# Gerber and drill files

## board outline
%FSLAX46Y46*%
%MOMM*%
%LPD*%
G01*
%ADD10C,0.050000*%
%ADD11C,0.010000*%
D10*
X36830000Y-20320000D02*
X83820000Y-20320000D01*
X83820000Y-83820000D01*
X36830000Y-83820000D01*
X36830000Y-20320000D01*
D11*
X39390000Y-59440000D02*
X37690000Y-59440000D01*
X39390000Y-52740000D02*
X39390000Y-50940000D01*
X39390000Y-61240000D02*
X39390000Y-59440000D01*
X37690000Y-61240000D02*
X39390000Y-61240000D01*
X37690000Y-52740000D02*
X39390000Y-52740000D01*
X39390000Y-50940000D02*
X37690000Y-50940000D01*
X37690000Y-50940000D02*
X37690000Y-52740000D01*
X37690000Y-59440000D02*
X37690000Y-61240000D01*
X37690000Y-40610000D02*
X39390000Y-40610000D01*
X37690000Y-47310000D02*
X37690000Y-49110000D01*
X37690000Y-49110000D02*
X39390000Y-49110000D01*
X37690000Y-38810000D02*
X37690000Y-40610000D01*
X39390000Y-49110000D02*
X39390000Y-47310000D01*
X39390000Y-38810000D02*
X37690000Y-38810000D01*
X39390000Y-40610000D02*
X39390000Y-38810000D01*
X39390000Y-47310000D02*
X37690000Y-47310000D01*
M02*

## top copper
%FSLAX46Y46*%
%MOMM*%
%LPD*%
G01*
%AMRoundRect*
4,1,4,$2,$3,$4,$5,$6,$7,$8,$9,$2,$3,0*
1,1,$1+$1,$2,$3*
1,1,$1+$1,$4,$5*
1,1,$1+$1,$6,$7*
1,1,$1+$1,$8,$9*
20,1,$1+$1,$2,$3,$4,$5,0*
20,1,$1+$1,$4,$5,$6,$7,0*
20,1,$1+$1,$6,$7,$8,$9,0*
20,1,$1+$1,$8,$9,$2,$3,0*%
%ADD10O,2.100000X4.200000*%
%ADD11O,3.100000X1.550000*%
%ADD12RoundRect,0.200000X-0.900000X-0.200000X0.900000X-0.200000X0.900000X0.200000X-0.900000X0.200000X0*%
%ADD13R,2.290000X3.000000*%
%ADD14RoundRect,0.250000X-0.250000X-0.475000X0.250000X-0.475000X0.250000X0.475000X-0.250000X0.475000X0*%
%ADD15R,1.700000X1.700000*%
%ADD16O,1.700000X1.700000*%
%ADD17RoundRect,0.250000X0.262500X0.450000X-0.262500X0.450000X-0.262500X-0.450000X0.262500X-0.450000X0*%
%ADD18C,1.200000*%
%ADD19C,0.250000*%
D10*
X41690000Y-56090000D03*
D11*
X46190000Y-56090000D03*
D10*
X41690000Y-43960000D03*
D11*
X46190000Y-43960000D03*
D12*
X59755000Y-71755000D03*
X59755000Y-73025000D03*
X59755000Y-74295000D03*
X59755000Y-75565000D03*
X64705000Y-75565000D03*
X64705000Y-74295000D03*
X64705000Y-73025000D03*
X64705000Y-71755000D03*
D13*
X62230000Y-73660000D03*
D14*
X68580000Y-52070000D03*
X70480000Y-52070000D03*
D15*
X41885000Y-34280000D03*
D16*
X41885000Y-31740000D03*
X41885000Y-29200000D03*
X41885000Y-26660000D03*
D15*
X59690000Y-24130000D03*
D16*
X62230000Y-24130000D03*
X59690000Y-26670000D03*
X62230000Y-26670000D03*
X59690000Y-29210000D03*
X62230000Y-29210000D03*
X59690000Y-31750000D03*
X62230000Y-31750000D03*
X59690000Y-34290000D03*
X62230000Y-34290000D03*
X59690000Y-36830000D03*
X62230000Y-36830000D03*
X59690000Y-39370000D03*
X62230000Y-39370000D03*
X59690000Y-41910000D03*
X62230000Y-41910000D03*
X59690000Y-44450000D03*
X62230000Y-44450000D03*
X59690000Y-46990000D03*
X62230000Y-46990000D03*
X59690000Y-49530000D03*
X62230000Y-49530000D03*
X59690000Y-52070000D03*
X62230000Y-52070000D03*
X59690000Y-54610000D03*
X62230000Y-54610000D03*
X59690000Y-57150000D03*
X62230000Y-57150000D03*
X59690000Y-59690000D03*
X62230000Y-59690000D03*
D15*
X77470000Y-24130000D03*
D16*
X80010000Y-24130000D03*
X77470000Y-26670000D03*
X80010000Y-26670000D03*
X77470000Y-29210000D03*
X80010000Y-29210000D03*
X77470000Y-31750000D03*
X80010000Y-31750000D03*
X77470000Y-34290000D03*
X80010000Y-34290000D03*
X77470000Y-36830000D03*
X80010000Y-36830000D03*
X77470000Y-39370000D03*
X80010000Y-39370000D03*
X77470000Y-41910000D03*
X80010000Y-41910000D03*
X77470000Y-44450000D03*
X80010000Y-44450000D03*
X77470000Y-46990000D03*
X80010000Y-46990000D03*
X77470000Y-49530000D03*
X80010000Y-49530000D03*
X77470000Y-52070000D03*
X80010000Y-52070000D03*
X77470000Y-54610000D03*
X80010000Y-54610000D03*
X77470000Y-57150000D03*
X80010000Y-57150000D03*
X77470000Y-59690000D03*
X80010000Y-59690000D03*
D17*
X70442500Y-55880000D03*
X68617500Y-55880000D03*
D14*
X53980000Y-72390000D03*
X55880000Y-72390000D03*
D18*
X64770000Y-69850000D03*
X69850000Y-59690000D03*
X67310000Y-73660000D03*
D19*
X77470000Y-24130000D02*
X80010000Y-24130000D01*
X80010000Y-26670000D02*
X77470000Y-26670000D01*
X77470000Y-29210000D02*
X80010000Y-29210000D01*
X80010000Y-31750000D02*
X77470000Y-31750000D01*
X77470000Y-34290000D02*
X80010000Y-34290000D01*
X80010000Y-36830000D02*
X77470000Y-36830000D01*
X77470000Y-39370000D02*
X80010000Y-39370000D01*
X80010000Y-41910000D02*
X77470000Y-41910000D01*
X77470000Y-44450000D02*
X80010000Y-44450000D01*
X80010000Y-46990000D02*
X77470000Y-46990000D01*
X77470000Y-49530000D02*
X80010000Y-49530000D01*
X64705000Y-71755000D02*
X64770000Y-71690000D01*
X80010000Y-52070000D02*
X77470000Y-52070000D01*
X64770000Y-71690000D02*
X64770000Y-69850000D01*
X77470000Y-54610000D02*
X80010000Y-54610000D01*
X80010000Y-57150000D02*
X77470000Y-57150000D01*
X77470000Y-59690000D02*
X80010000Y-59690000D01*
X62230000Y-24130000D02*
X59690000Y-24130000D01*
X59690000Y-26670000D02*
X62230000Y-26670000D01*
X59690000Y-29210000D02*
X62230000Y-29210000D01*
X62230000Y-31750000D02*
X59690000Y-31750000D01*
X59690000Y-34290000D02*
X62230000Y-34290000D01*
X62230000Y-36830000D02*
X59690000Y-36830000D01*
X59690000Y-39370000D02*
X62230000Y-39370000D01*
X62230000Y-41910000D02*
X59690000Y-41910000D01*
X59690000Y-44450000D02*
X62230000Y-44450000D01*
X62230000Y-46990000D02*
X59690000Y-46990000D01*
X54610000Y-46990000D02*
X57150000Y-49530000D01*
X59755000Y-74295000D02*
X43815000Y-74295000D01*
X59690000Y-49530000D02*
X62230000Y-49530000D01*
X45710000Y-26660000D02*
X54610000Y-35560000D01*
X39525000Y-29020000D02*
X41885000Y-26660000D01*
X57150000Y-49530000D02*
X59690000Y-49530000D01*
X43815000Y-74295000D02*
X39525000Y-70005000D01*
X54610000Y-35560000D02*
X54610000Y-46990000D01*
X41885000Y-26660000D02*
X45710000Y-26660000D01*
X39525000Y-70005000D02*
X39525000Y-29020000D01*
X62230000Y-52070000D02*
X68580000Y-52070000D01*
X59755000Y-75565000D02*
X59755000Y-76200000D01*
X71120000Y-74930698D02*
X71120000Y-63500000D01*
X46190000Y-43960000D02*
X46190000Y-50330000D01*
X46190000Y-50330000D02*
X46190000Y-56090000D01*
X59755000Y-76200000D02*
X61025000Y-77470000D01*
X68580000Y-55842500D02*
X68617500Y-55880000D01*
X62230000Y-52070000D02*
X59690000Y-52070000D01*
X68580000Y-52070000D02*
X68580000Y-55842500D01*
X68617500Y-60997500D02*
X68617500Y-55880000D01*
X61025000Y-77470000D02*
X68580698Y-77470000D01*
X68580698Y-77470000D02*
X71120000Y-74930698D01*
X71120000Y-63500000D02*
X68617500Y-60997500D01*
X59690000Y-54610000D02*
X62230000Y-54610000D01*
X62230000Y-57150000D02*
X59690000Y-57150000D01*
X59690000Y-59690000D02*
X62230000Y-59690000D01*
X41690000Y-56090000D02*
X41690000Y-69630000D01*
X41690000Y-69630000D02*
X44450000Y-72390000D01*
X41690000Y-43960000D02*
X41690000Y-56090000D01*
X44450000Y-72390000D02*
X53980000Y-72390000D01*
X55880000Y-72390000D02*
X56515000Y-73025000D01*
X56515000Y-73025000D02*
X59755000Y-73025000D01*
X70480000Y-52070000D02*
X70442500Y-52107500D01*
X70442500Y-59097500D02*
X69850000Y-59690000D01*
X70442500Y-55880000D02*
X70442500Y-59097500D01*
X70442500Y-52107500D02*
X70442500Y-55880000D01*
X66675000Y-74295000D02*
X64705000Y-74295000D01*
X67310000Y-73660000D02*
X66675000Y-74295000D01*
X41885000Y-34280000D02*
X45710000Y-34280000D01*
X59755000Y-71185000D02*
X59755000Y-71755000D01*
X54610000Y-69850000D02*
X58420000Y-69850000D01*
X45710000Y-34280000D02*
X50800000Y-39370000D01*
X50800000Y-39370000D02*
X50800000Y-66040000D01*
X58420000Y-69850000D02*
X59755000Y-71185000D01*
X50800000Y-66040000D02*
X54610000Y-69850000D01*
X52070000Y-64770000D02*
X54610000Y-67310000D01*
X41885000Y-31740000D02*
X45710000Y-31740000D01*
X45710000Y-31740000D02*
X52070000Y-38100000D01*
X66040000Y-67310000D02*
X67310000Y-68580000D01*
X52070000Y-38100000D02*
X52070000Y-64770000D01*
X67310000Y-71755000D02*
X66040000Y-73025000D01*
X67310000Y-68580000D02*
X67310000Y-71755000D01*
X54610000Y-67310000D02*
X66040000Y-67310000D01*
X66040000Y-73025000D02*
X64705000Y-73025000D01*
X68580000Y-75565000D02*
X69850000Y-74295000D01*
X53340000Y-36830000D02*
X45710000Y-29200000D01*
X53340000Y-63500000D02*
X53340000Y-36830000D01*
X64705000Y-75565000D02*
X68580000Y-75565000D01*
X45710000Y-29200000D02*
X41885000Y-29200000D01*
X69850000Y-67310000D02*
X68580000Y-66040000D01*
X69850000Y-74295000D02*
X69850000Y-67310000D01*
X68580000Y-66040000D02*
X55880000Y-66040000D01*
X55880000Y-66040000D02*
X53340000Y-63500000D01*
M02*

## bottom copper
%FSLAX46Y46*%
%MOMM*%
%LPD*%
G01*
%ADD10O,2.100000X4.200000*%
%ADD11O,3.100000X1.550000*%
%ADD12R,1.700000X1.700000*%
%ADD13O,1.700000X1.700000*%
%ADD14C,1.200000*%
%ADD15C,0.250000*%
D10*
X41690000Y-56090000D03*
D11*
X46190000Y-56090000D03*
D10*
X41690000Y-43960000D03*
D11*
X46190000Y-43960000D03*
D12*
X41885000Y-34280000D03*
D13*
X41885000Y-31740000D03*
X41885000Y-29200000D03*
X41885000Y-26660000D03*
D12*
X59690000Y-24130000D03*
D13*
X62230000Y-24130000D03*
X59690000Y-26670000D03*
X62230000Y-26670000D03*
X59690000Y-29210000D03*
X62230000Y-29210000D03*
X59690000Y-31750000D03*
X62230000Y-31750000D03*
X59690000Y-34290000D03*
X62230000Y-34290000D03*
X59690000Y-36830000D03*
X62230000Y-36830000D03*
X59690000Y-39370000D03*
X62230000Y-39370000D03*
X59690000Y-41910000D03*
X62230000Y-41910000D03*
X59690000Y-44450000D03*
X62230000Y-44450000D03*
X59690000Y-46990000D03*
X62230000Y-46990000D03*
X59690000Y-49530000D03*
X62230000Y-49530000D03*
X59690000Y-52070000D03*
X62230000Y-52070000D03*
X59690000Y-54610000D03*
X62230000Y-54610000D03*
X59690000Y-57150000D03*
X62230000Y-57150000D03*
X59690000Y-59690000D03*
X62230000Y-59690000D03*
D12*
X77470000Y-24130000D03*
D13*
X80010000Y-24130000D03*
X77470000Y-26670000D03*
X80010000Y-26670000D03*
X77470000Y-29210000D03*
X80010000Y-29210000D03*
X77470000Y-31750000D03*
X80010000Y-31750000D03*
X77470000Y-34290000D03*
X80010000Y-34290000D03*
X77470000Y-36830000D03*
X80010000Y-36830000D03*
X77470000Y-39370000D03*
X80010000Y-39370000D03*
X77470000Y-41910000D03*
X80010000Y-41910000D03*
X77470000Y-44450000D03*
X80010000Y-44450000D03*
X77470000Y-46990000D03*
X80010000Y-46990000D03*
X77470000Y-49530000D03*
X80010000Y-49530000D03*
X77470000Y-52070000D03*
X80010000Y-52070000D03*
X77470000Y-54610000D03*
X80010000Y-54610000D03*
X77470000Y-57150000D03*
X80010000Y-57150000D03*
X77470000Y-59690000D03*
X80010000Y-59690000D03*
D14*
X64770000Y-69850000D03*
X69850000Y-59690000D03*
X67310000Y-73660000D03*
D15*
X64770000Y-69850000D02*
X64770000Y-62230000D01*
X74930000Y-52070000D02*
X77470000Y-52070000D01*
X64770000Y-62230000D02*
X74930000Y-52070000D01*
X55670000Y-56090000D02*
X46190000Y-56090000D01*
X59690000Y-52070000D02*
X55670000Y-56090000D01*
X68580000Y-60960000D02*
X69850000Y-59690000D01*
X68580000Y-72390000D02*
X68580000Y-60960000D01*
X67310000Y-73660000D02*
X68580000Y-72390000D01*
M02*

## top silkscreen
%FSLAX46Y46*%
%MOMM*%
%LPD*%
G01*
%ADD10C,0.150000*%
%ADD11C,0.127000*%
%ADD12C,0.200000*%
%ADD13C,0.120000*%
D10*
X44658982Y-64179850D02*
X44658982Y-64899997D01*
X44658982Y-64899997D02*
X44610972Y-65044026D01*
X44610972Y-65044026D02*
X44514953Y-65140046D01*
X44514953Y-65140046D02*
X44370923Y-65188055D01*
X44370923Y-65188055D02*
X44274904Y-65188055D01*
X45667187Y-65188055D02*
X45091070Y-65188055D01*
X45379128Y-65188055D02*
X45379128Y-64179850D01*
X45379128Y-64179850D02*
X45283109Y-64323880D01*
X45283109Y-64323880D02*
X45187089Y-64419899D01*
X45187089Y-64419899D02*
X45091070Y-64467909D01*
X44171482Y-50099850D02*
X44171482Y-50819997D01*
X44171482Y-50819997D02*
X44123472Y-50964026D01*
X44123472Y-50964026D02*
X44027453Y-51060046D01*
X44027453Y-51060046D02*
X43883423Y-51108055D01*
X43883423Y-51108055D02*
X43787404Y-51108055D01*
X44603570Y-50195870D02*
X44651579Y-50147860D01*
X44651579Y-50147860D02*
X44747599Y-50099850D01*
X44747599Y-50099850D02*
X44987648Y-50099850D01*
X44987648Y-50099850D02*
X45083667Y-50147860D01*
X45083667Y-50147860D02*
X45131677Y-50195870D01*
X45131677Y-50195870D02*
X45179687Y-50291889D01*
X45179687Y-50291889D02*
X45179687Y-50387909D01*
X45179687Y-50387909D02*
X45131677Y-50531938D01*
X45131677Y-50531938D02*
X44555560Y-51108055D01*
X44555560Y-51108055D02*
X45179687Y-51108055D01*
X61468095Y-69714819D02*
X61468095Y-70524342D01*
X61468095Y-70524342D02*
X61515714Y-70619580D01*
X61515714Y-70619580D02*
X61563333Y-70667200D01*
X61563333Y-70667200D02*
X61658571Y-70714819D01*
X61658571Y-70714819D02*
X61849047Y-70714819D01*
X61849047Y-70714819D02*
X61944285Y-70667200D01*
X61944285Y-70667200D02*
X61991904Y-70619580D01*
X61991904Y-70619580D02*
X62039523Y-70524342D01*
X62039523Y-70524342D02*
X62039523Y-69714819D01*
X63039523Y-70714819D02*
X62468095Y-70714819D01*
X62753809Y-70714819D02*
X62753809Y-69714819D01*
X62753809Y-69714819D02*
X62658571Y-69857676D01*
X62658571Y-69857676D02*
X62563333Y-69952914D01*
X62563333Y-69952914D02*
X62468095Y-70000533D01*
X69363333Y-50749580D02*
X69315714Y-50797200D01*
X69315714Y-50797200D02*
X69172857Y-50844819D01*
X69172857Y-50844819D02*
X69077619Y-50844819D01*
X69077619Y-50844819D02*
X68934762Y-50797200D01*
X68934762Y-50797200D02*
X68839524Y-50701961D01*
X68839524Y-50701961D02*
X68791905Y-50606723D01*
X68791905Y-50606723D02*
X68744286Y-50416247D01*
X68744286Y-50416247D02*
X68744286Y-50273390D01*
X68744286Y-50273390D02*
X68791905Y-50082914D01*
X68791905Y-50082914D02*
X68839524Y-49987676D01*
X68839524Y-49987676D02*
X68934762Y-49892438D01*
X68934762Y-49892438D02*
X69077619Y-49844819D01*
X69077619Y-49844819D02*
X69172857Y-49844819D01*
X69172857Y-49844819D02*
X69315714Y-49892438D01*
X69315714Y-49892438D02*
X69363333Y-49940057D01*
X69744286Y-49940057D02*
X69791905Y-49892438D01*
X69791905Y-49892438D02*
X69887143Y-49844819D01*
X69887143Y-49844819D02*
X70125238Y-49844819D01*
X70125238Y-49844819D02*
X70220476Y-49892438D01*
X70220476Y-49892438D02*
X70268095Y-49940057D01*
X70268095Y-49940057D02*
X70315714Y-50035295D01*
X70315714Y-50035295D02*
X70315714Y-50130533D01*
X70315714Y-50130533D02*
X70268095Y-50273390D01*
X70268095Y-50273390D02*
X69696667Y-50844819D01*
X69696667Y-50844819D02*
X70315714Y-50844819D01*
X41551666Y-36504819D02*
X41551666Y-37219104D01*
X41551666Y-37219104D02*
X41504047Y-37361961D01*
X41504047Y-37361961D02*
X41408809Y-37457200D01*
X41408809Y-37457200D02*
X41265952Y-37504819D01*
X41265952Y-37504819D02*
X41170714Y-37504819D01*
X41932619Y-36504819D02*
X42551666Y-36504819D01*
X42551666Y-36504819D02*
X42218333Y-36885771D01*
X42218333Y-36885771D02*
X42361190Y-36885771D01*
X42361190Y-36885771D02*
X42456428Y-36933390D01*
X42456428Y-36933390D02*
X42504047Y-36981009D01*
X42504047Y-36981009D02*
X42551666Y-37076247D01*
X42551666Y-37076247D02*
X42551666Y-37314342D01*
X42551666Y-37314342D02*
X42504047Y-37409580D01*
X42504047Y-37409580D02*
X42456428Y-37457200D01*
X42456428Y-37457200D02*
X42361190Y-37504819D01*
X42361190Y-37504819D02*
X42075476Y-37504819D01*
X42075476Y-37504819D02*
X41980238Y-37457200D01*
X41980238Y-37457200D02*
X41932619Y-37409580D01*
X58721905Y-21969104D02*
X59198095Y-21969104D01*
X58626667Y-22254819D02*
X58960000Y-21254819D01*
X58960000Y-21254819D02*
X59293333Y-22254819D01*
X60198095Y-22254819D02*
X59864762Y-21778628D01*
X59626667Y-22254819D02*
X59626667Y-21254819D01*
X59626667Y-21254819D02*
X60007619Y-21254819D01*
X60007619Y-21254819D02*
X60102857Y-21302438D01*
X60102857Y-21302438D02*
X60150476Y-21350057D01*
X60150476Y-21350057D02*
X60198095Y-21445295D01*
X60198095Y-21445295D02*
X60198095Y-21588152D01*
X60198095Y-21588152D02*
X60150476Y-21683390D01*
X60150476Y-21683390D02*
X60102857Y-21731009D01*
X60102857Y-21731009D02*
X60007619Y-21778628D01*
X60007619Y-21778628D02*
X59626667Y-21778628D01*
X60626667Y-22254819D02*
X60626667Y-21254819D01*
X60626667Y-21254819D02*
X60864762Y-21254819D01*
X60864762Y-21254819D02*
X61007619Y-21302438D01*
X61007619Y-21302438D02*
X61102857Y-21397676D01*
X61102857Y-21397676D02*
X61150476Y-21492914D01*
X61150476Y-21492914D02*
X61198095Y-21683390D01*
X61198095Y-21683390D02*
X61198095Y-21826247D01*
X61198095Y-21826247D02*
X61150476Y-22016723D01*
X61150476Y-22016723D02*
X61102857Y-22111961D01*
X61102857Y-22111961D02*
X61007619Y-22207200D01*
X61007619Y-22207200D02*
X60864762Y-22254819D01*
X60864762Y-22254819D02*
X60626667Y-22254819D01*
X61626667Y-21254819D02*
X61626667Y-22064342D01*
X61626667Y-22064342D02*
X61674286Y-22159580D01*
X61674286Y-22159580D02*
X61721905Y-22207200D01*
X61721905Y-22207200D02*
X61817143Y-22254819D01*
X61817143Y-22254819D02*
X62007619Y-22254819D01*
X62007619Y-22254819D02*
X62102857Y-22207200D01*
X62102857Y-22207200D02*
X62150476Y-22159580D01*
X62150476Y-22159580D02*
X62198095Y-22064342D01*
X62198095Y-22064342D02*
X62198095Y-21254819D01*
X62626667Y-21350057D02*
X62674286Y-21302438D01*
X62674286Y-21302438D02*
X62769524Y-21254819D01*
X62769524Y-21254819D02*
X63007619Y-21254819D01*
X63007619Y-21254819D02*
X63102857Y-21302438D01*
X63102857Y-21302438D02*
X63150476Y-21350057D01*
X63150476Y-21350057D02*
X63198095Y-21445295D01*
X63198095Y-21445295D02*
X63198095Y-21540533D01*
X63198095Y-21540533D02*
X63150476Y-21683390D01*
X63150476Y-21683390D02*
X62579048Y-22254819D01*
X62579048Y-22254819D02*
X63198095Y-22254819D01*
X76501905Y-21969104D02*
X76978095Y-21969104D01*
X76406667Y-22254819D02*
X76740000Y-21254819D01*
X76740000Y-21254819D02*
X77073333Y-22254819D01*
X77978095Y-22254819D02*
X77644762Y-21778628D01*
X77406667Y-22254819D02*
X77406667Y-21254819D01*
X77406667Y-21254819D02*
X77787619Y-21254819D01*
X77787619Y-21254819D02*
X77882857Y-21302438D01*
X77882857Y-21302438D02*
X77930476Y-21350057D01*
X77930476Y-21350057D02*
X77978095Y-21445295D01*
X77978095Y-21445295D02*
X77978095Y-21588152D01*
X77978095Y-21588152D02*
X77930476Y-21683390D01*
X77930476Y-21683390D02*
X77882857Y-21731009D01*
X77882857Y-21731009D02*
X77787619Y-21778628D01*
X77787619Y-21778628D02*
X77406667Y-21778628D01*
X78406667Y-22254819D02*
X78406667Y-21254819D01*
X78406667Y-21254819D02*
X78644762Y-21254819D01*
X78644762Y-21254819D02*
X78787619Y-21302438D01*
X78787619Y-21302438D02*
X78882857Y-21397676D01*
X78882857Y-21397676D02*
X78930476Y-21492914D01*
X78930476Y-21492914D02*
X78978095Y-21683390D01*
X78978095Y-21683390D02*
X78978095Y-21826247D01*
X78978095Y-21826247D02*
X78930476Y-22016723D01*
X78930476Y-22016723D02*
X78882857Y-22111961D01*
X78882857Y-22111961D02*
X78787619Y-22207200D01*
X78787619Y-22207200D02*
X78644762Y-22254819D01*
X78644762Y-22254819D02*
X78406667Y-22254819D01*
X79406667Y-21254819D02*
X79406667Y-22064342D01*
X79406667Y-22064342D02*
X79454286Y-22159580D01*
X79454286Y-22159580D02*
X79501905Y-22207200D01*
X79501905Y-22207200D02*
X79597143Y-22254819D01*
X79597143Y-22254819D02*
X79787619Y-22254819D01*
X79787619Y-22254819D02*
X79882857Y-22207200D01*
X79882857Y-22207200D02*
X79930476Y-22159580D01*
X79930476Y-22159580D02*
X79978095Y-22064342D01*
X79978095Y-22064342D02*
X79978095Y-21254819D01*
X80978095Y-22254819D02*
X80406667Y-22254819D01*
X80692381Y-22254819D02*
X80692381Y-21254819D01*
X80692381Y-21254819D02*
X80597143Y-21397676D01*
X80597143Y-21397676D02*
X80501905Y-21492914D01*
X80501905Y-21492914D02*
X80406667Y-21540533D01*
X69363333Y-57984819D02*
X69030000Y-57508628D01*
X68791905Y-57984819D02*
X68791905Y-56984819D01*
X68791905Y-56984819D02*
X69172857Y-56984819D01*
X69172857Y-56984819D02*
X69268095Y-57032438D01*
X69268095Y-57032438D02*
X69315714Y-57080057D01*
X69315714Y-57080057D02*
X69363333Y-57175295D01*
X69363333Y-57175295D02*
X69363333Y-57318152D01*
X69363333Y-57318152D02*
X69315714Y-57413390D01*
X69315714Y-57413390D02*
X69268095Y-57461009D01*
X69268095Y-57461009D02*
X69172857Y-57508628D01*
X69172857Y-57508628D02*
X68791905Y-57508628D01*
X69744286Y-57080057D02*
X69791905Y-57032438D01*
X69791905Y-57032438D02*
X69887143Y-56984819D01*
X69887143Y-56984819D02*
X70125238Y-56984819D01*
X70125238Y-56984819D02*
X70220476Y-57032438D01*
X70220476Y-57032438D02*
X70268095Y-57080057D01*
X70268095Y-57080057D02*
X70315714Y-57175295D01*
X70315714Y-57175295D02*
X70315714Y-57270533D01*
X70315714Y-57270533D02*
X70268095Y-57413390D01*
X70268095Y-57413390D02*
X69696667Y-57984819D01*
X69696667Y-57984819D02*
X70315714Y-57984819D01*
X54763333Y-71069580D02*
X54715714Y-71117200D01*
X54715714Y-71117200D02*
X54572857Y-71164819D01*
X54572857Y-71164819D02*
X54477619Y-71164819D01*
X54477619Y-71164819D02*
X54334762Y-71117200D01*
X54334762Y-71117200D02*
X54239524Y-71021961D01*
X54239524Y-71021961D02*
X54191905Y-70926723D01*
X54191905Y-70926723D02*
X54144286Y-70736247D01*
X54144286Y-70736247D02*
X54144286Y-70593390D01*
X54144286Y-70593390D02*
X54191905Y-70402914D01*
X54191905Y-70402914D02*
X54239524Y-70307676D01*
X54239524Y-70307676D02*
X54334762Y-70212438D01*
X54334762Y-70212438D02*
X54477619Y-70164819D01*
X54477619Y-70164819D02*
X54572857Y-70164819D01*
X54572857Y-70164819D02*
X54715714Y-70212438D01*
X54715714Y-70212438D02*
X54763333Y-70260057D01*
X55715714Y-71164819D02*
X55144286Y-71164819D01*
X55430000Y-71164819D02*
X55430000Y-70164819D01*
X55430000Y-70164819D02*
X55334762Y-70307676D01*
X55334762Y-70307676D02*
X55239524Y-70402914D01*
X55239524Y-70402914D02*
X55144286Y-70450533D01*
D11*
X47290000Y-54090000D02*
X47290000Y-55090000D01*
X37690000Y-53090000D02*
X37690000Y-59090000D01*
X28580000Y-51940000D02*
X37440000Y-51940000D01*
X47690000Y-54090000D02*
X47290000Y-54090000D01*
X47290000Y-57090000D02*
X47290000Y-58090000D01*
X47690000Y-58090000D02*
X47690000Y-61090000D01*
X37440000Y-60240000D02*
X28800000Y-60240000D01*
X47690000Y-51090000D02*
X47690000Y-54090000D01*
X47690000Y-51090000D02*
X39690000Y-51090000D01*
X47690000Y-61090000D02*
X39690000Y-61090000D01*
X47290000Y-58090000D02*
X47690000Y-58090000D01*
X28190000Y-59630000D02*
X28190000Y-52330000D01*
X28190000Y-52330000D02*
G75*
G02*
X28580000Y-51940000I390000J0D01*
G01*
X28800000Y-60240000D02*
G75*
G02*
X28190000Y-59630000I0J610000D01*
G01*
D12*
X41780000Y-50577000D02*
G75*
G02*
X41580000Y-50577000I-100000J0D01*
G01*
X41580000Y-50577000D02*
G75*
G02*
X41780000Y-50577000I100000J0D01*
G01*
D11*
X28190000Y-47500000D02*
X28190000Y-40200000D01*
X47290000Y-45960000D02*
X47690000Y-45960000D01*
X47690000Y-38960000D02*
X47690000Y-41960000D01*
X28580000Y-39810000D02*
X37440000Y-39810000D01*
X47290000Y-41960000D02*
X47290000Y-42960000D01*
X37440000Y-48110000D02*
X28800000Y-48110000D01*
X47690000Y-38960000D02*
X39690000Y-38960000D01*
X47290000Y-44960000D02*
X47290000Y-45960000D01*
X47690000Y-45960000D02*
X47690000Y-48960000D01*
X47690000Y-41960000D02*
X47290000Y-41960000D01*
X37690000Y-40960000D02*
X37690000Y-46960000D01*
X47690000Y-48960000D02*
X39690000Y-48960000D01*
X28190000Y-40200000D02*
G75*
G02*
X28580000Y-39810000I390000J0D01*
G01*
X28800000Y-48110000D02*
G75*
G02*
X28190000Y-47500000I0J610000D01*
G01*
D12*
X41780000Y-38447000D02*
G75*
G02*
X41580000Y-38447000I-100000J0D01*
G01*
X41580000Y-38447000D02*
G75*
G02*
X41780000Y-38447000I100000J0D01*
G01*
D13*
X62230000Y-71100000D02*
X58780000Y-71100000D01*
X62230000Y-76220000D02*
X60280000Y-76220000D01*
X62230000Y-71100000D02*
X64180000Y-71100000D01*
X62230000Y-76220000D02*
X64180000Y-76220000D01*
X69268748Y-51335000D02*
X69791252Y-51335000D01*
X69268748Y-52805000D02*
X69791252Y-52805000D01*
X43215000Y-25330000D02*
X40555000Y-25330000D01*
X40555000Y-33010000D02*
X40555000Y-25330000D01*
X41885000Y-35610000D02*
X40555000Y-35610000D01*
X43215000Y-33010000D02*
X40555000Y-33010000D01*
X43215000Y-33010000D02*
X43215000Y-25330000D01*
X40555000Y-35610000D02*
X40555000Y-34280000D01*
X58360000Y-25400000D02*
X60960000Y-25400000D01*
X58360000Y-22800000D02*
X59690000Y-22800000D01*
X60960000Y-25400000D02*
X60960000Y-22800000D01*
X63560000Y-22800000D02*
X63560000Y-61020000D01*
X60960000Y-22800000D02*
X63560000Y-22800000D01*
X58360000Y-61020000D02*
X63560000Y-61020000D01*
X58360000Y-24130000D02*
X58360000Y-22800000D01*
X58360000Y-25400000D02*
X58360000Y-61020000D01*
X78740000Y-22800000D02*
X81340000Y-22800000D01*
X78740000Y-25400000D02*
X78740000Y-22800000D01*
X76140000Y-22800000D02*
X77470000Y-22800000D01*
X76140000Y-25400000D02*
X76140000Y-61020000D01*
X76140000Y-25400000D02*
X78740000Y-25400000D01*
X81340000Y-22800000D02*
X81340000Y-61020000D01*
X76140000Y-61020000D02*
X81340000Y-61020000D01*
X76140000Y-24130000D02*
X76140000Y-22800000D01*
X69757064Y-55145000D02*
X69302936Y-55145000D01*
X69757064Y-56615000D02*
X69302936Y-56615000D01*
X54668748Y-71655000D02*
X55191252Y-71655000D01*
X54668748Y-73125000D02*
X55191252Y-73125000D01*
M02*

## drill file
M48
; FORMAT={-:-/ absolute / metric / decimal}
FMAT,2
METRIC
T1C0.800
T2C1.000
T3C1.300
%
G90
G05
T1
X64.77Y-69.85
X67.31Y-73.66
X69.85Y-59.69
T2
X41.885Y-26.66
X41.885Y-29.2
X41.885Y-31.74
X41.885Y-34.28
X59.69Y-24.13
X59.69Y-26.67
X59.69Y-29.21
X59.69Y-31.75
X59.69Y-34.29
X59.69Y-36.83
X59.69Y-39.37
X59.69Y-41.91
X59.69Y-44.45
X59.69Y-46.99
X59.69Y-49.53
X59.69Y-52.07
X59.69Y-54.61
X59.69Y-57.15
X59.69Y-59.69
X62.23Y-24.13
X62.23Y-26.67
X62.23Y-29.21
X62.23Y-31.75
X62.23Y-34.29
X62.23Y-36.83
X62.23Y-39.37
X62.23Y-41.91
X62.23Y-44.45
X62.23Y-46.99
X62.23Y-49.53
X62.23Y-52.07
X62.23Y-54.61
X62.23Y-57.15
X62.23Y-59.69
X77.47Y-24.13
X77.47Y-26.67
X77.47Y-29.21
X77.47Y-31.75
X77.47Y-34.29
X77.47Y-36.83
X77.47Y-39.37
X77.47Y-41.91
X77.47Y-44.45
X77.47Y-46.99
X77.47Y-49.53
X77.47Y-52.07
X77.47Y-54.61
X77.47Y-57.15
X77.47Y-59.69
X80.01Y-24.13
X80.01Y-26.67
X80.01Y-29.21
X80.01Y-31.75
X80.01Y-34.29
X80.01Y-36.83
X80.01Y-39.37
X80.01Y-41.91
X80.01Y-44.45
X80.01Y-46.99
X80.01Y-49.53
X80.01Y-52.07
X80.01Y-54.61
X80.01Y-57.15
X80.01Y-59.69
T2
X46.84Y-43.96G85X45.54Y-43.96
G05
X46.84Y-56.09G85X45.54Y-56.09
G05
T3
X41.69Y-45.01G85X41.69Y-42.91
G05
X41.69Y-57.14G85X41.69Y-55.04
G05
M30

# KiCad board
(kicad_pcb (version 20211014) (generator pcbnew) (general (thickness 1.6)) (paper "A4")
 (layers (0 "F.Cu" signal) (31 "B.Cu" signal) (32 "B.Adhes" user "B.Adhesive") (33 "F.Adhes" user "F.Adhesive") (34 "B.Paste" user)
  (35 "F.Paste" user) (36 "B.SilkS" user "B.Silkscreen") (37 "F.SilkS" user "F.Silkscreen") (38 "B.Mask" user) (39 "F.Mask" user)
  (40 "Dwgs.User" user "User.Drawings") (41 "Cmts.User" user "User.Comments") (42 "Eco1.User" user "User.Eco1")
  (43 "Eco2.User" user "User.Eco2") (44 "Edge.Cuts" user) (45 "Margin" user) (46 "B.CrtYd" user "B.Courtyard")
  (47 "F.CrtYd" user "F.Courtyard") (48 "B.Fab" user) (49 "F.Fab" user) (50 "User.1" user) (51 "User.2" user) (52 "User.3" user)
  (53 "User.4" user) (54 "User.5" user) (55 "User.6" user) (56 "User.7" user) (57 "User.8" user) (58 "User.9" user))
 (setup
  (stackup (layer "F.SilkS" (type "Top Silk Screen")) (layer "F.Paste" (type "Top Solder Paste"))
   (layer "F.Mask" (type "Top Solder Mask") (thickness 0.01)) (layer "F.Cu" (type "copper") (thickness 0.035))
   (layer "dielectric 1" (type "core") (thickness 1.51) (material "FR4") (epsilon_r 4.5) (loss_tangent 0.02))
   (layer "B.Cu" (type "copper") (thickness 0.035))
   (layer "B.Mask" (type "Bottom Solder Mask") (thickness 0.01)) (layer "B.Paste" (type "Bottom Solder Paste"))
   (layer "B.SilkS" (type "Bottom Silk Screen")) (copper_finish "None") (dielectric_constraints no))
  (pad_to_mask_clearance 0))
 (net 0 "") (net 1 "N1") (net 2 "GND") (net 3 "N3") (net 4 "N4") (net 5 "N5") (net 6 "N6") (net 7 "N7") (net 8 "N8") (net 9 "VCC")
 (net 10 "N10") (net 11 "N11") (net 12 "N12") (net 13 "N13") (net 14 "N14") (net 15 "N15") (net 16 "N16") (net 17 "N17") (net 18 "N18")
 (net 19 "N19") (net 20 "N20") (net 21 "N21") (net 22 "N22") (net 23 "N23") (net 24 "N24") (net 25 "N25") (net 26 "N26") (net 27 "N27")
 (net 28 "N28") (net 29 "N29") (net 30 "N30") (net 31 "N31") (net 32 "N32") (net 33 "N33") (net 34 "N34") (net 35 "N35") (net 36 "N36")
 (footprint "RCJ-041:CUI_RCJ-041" (layer "F.Cu") (at 37.69 56.09 180)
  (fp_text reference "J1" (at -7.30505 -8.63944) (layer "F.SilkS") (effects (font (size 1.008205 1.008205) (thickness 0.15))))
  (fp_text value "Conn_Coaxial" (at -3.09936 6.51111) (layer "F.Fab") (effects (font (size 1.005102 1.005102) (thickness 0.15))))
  (fp_line (start -9.6 2) (end -9.6 1) (layer "F.SilkS") (width 0.127))
  (fp_line (start 0 3) (end 0 -3) (layer "F.SilkS") (width 0.127))
  (fp_line (start 9.11 4.15) (end 0.25 4.15) (layer "F.SilkS") (width 0.127))
  (fp_line (start -10 2) (end -9.6 2) (layer "F.SilkS") (width 0.127))
  (fp_line (start -9.6 -1) (end -9.6 -2) (layer "F.SilkS") (width 0.127))
  (fp_line (start -10 -2) (end -10 -5) (layer "F.SilkS") (width 0.127))
  (fp_line (start 0.25 -4.15) (end 8.89 -4.15) (layer "F.SilkS") (width 0.127))
  (fp_line (start -10 5) (end -10 2) (layer "F.SilkS") (width 0.127))
  (fp_line (start -10 5) (end -2 5) (layer "F.SilkS") (width 0.127))
  (fp_line (start -10 -5) (end -2 -5) (layer "F.SilkS") (width 0.127))
  (fp_line (start -9.6 -2) (end -10 -2) (layer "F.SilkS") (width 0.127))
  (fp_line (start 9.5 -3.54) (end 9.5 3.76) (layer "F.SilkS") (width 0.127))
  (fp_arc (start 9.5 3.76) (mid 9.385772 4.035772) (end 9.11 4.15) (layer "F.SilkS") (width 0.127))
  (fp_arc (start 8.89 -4.15) (mid 9.321335 -3.971335) (end 9.5 -3.54) (layer "F.SilkS") (width 0.127))
  (fp_circle (center -3.99 5.513) (end -3.89 5.513) (layer "F.SilkS") (width 0.2) (fill none))
  (fp_line (start -1.7 -3.35) (end 0 -3.35) (layer "Edge.Cuts") (width 0.01))
  (fp_line (start -1.7 3.35) (end -1.7 5.15) (layer "Edge.Cuts") (width 0.01))
  (fp_line (start -1.7 -5.15) (end -1.7 -3.35) (layer "Edge.Cuts") (width 0.01))
  (fp_line (start 0 -5.15) (end -1.7 -5.15) (layer "Edge.Cuts") (width 0.01))
  (fp_line (start 0 3.35) (end -1.7 3.35) (layer "Edge.Cuts") (width 0.01))
  (fp_line (start -1.7 5.15) (end 0 5.15) (layer "Edge.Cuts") (width 0.01))
  (fp_line (start 0 5.15) (end 0 3.35) (layer "Edge.Cuts") (width 0.01))
  (fp_line (start 0 -3.35) (end 0 -5.15) (layer "Edge.Cuts") (width 0.01))
  (pad "1" thru_hole oval locked (at -4 0 180) (size 2.1 4.2) (drill oval 1.3 3.4) (layers *.Cu *.Mask) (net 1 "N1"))
  (pad "2" thru_hole oval locked (at -8.5 0 180) (size 3.1 1.55) (drill oval 2.3 1) (layers *.Cu *.Mask) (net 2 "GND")))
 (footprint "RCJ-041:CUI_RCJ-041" (layer "F.Cu") (at 37.69 43.96 180)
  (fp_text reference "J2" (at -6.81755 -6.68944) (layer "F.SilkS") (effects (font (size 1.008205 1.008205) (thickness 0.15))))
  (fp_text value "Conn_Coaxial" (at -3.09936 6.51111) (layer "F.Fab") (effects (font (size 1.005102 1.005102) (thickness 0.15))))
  (fp_line (start 9.5 -3.54) (end 9.5 3.76) (layer "F.SilkS") (width 0.127))
  (fp_line (start -9.6 -2) (end -10 -2) (layer "F.SilkS") (width 0.127))
  (fp_line (start -10 5) (end -10 2) (layer "F.SilkS") (width 0.127))
  (fp_line (start 9.11 4.15) (end 0.25 4.15) (layer "F.SilkS") (width 0.127))
  (fp_line (start -9.6 2) (end -9.6 1) (layer "F.SilkS") (width 0.127))
  (fp_line (start 0.25 -4.15) (end 8.89 -4.15) (layer "F.SilkS") (width 0.127))
  (fp_line (start -10 5) (end -2 5) (layer "F.SilkS") (width 0.127))
  (fp_line (start -9.6 -1) (end -9.6 -2) (layer "F.SilkS") (width 0.127))
  (fp_line (start -10 -2) (end -10 -5) (layer "F.SilkS") (width 0.127))
  (fp_line (start -10 2) (end -9.6 2) (layer "F.SilkS") (width 0.127))
  (fp_line (start 0 3) (end 0 -3) (layer "F.SilkS") (width 0.127))
  (fp_line (start -10 -5) (end -2 -5) (layer "F.SilkS") (width 0.127))
  (fp_arc (start 9.5 3.76) (mid 9.385772 4.035772) (end 9.11 4.15) (layer "F.SilkS") (width 0.127))
  (fp_arc (start 8.89 -4.15) (mid 9.321335 -3.971335) (end 9.5 -3.54) (layer "F.SilkS") (width 0.127))
  (fp_circle (center -3.99 5.513) (end -3.89 5.513) (layer "F.SilkS") (width 0.2) (fill none))
  (fp_line (start 0 3.35) (end -1.7 3.35) (layer "Edge.Cuts") (width 0.01))
  (fp_line (start 0 -3.35) (end 0 -5.15) (layer "Edge.Cuts") (width 0.01))
  (fp_line (start 0 -5.15) (end -1.7 -5.15) (layer "Edge.Cuts") (width 0.01))
  (fp_line (start 0 5.15) (end 0 3.35) (layer "Edge.Cuts") (width 0.01))
  (fp_line (start -1.7 -5.15) (end -1.7 -3.35) (layer "Edge.Cuts") (width 0.01))
  (fp_line (start -1.7 5.15) (end 0 5.15) (layer "Edge.Cuts") (width 0.01))
  (fp_line (start -1.7 3.35) (end -1.7 5.15) (layer "Edge.Cuts") (width 0.01))
  (fp_line (start -1.7 -3.35) (end 0 -3.35) (layer "Edge.Cuts") (width 0.01))
  (pad "1" thru_hole oval locked (at -4 0 180) (size 2.1 4.2) (drill oval 1.3 3.4) (layers *.Cu *.Mask) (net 1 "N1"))
  (pad "2" thru_hole oval locked (at -8.5 0 180) (size 3.1 1.55) (drill oval 2.3 1) (layers *.Cu *.Mask) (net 2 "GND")))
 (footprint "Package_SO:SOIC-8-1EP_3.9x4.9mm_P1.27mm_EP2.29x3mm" (layer "F.Cu") (at 62.23 73.66)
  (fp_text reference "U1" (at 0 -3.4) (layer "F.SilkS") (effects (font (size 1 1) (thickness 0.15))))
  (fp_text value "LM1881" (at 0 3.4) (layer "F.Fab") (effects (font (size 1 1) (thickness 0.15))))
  (fp_line (start 0 -2.56) (end -3.45 -2.56) (layer "F.SilkS") (width 0.12))
  (fp_line (start 0 2.56) (end -1.95 2.56) (layer "F.SilkS") (width 0.12))
  (fp_line (start 0 -2.56) (end 1.95 -2.56) (layer "F.SilkS") (width 0.12))
  (fp_line (start 0 2.56) (end 1.95 2.56) (layer "F.SilkS") (width 0.12))
  (pad "" smd roundrect (at 0.57 -0.75) (size 0.92 1.21) (layers "F.Paste") (roundrect_rratio 0.25))
  (pad "" smd roundrect (at -0.57 0.75) (size 0.92 1.21) (layers "F.Paste") (roundrect_rratio 0.25))
  (pad "" smd roundrect (at -0.57 -0.75) (size 0.92 1.21) (layers "F.Paste") (roundrect_rratio 0.25))
  (pad "" smd roundrect (at 0.57 0.75) (size 0.92 1.21) (layers "F.Paste") (roundrect_rratio 0.25))
  (pad "1" smd roundrect (at -2.475 -1.905) (size 2.2 0.8) (layers "F.Cu" "F.Paste" "F.Mask") (roundrect_rratio 0.25) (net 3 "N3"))
  (pad "2" smd roundrect (at -2.475 -0.635) (size 2.2 0.8) (layers "F.Cu" "F.Paste" "F.Mask") (roundrect_rratio 0.25) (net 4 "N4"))
  (pad "3" smd roundrect (at -2.475 0.635) (size 2.2 0.8) (layers "F.Cu" "F.Paste" "F.Mask") (roundrect_rratio 0.25) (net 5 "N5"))
  (pad "4" smd roundrect (at -2.475 1.905) (size 2.2 0.8) (layers "F.Cu" "F.Paste" "F.Mask") (roundrect_rratio 0.25) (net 2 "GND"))
  (pad "5" smd roundrect (at 2.475 1.905) (size 2.2 0.8) (layers "F.Cu" "F.Paste" "F.Mask") (roundrect_rratio 0.25) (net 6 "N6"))
  (pad "6" smd roundrect (at 2.475 0.635) (size 2.2 0.8) (layers "F.Cu" "F.Paste" "F.Mask") (roundrect_rratio 0.25) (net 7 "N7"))
  (pad "7" smd roundrect (at 2.475 -0.635) (size 2.2 0.8) (layers "F.Cu" "F.Paste" "F.Mask") (roundrect_rratio 0.25) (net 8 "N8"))
  (pad "8" smd roundrect (at 2.475 -1.905) (size 2.2 0.8) (layers "F.Cu" "F.Paste" "F.Mask") (roundrect_rratio 0.25) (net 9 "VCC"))
  (pad "9" smd rect (at 0 0) (size 2.29 3) (layers "F.Cu" "F.Mask")))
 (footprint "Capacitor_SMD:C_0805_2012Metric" (layer "F.Cu") (at 69.53 52.07)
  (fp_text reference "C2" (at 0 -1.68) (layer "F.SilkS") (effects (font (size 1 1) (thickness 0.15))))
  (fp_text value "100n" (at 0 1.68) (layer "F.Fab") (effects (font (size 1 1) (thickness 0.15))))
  (fp_line (start -0.261252 -0.735) (end 0.261252 -0.735) (layer "F.SilkS") (width 0.12))
  (fp_line (start -0.261252 0.735) (end 0.261252 0.735) (layer "F.SilkS") (width 0.12))
  (pad "1" smd roundrect (at -0.95 0) (size 1 1.45) (layers "F.Cu" "F.Paste" "F.Mask") (roundrect_rratio 0.25) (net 2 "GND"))
  (pad "2" smd roundrect (at 0.95 0) (size 1 1.45) (layers "F.Cu" "F.Paste" "F.Mask") (roundrect_rratio 0.25) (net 7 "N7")))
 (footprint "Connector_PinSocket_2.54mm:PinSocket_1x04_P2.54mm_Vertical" (layer "F.Cu") (at 41.885 34.28 180)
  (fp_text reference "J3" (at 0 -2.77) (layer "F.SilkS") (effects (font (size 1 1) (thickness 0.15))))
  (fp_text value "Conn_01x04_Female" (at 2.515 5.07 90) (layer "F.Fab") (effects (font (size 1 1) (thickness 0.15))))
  (fp_line (start -1.33 8.95) (end 1.33 8.95) (layer "F.SilkS") (width 0.12))
  (fp_line (start 1.33 1.27) (end 1.33 8.95) (layer "F.SilkS") (width 0.12))
  (fp_line (start 0 -1.33) (end 1.33 -1.33) (layer "F.SilkS") (width 0.12))
  (fp_line (start -1.33 1.27) (end 1.33 1.27) (layer "F.SilkS") (width 0.12))
  (fp_line (start -1.33 1.27) (end -1.33 8.95) (layer "F.SilkS") (width 0.12))
  (fp_line (start 1.33 -1.33) (end 1.33 0) (layer "F.SilkS") (width 0.12))
  (pad "1" thru_hole rect (at 0 0 180) (size 1.7 1.7) (drill 1) (layers *.Cu *.Mask) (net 3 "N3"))
  (pad "2" thru_hole oval (at 0 2.54 180) (size 1.7 1.7) (drill 1) (layers *.Cu *.Mask) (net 8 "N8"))
  (pad "3" thru_hole oval (at 0 5.08 180) (size 1.7 1.7) (drill 1) (layers *.Cu *.Mask) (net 6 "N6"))
  (pad "4" thru_hole oval (at 0 7.62 180) (size 1.7 1.7) (drill 1) (layers *.Cu *.Mask) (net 5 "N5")))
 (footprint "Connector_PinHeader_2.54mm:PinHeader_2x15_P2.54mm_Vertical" (layer "F.Cu") (at 59.69 24.13)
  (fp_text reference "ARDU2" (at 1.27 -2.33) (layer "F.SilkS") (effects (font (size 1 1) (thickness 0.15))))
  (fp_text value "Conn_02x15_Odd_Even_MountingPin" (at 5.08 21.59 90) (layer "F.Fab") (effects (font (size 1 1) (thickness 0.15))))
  (fp_line (start -1.33 1.27) (end 1.27 1.27) (layer "F.SilkS") (width 0.12))
  (fp_line (start -1.33 -1.33) (end 0 -1.33) (layer "F.SilkS") (width 0.12))
  (fp_line (start 1.27 1.27) (end 1.27 -1.33) (layer "F.SilkS") (width 0.12))
  (fp_line (start 3.87 -1.33) (end 3.87 36.89) (layer "F.SilkS") (width 0.12))
  (fp_line (start 1.27 -1.33) (end 3.87 -1.33) (layer "F.SilkS") (width 0.12))
  (fp_line (start -1.33 36.89) (end 3.87 36.89) (layer "F.SilkS") (width 0.12))
  (fp_line (start -1.33 0) (end -1.33 -1.33) (layer "F.SilkS") (width 0.12))
  (fp_line (start -1.33 1.27) (end -1.33 36.89) (layer "F.SilkS") (width 0.12))
  (pad "1" thru_hole rect (at 0 0) (size 1.7 1.7) (drill 1) (layers *.Cu *.Mask) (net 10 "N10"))
  (pad "2" thru_hole oval (at 2.54 0) (size 1.7 1.7) (drill 1) (layers *.Cu *.Mask) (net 10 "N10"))
  (pad "3" thru_hole oval (at 0 2.54) (size 1.7 1.7) (drill 1) (layers *.Cu *.Mask) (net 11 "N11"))
  (pad "4" thru_hole oval (at 2.54 2.54) (size 1.7 1.7) (drill 1) (layers *.Cu *.Mask) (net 11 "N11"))
  (pad "5" thru_hole oval (at 0 5.08) (size 1.7 1.7) (drill 1) (layers *.Cu *.Mask) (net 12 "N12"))
  (pad "6" thru_hole oval (at 2.54 5.08) (size 1.7 1.7) (drill 1) (layers *.Cu *.Mask) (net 12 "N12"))
  (pad "7" thru_hole oval (at 0 7.62) (size 1.7 1.7) (drill 1) (layers *.Cu *.Mask) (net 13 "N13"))
  (pad "8" thru_hole oval (at 2.54 7.62) (size 1.7 1.7) (drill 1) (layers *.Cu *.Mask) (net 13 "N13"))
  (pad "9" thru_hole oval (at 0 10.16) (size 1.7 1.7) (drill 1) (layers *.Cu *.Mask) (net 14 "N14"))
  (pad "10" thru_hole oval (at 2.54 10.16) (size 1.7 1.7) (drill 1) (layers *.Cu *.Mask) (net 14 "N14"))
  (pad "11" thru_hole oval (at 0 12.7) (size 1.7 1.7) (drill 1) (layers *.Cu *.Mask) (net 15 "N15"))
  (pad "12" thru_hole oval (at 2.54 12.7) (size 1.7 1.7) (drill 1) (layers *.Cu *.Mask) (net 15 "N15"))
  (pad "13" thru_hole oval (at 0 15.24) (size 1.7 1.7) (drill 1) (layers *.Cu *.Mask) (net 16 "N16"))
  (pad "14" thru_hole oval (at 2.54 15.24) (size 1.7 1.7) (drill 1) (layers *.Cu *.Mask) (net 16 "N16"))
  (pad "15" thru_hole oval (at 0 17.78) (size 1.7 1.7) (drill 1) (layers *.Cu *.Mask) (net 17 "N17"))
  (pad "16" thru_hole oval (at 2.54 17.78) (size 1.7 1.7) (drill 1) (layers *.Cu *.Mask) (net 17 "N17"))
  (pad "17" thru_hole oval (at 0 20.32) (size 1.7 1.7) (drill 1) (layers *.Cu *.Mask) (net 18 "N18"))
  (pad "18" thru_hole oval (at 2.54 20.32) (size 1.7 1.7) (drill 1) (layers *.Cu *.Mask) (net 18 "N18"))
  (pad "19" thru_hole oval (at 0 22.86) (size 1.7 1.7) (drill 1) (layers *.Cu *.Mask) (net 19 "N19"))
  (pad "20" thru_hole oval (at 2.54 22.86) (size 1.7 1.7) (drill 1) (layers *.Cu *.Mask) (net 19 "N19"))
  (pad "21" thru_hole oval (at 0 25.4) (size 1.7 1.7) (drill 1) (layers *.Cu *.Mask) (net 5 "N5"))
  (pad "22" thru_hole oval (at 2.54 25.4) (size 1.7 1.7) (drill 1) (layers *.Cu *.Mask) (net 5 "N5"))
  (pad "23" thru_hole oval (at 0 27.94) (size 1.7 1.7) (drill 1) (layers *.Cu *.Mask) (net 2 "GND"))
  (pad "24" thru_hole oval (at 2.54 27.94) (size 1.7 1.7) (drill 1) (layers *.Cu *.Mask) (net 2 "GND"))
  (pad "25" thru_hole oval (at 0 30.48) (size 1.7 1.7) (drill 1) (layers *.Cu *.Mask) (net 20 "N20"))
  (pad "26" thru_hole oval (at 2.54 30.48) (size 1.7 1.7) (drill 1) (layers *.Cu *.Mask) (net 20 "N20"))
  (pad "27" thru_hole oval (at 0 33.02) (size 1.7 1.7) (drill 1) (layers *.Cu *.Mask) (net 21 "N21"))
  (pad "28" thru_hole oval (at 2.54 33.02) (size 1.7 1.7) (drill 1) (layers *.Cu *.Mask) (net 21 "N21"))
  (pad "29" thru_hole oval (at 0 35.56) (size 1.7 1.7) (drill 1) (layers *.Cu *.Mask) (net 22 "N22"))
  (pad "30" thru_hole oval (at 2.54 35.56) (size 1.7 1.7) (drill 1) (layers *.Cu *.Mask) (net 22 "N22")))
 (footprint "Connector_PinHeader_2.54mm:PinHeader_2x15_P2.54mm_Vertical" (layer "F.Cu") (at 77.47 24.13)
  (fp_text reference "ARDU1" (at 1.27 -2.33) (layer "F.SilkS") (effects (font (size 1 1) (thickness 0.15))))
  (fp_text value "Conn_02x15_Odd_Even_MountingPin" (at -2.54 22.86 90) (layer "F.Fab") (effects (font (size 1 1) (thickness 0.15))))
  (fp_line (start 1.27 -1.33) (end 3.87 -1.33) (layer "F.SilkS") (width 0.12))
  (fp_line (start 1.27 1.27) (end 1.27 -1.33) (layer "F.SilkS") (width 0.12))
  (fp_line (start -1.33 -1.33) (end 0 -1.33) (layer "F.SilkS") (width 0.12))
  (fp_line (start -1.33 1.27) (end -1.33 36.89) (layer "F.SilkS") (width 0.12))
  (fp_line (start -1.33 1.27) (end 1.27 1.27) (layer "F.SilkS") (width 0.12))
  (fp_line (start 3.87 -1.33) (end 3.87 36.89) (layer "F.SilkS") (width 0.12))
  (fp_line (start -1.33 36.89) (end 3.87 36.89) (layer "F.SilkS") (width 0.12))
  (fp_line (start -1.33 0) (end -1.33 -1.33) (layer "F.SilkS") (width 0.12))
  (pad "1" thru_hole rect (at 0 0) (size 1.7 1.7) (drill 1) (layers *.Cu *.Mask) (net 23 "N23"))
  (pad "2" thru_hole oval (at 2.54 0) (size 1.7 1.7) (drill 1) (layers *.Cu *.Mask) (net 23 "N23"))
  (pad "3" thru_hole oval (at 0 2.54) (size 1.7 1.7) (drill 1) (layers *.Cu *.Mask) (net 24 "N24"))
  (pad "4" thru_hole oval (at 2.54 2.54) (size 1.7 1.7) (drill 1) (layers *.Cu *.Mask) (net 24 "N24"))
  (pad "5" thru_hole oval (at 0 5.08) (size 1.7 1.7) (drill 1) (layers *.Cu *.Mask) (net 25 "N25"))
  (pad "6" thru_hole oval (at 2.54 5.08) (size 1.7 1.7) (drill 1) (layers *.Cu *.Mask) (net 25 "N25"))
  (pad "7" thru_hole oval (at 0 7.62) (size 1.7 1.7) (drill 1) (layers *.Cu *.Mask) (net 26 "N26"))
  (pad "8" thru_hole oval (at 2.54 7.62) (size 1.7 1.7) (drill 1) (layers *.Cu *.Mask) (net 26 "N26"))
  (pad "9" thru_hole oval (at 0 10.16) (size 1.7 1.7) (drill 1) (layers *.Cu *.Mask) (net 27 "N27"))
  (pad "10" thru_hole oval (at 2.54 10.16) (size 1.7 1.7) (drill 1) (layers *.Cu *.Mask) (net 27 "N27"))
  (pad "11" thru_hole oval (at 0 12.7) (size 1.7 1.7) (drill 1) (layers *.Cu *.Mask) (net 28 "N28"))
  (pad "12" thru_hole oval (at 2.54 12.7) (size 1.7 1.7) (drill 1) (layers *.Cu *.Mask) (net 28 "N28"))
  (pad "13" thru_hole oval (at 0 15.24) (size 1.7 1.7) (drill 1) (layers *.Cu *.Mask) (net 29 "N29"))
  (pad "14" thru_hole oval (at 2.54 15.24) (size 1.7 1.7) (drill 1) (layers *.Cu *.Mask) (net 29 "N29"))
  (pad "15" thru_hole oval (at 0 17.78) (size 1.7 1.7) (drill 1) (layers *.Cu *.Mask) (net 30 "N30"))
  (pad "16" thru_hole oval (at 2.54 17.78) (size 1.7 1.7) (drill 1) (layers *.Cu *.Mask) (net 30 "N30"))
  (pad "17" thru_hole oval (at 0 20.32) (size 1.7 1.7) (drill 1) (layers *.Cu *.Mask) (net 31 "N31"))
  (pad "18" thru_hole oval (at 2.54 20.32) (size 1.7 1.7) (drill 1) (layers *.Cu *.Mask) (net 31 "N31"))
  (pad "19" thru_hole oval (at 0 22.86) (size 1.7 1.7) (drill 1) (layers *.Cu *.Mask) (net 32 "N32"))
  (pad "20" thru_hole oval (at 2.54 22.86) (size 1.7 1.7) (drill 1) (layers *.Cu *.Mask) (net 32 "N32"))
  (pad "21" thru_hole oval (at 0 25.4) (size 1.7 1.7) (drill 1) (layers *.Cu *.Mask) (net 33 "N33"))
  (pad "22" thru_hole oval (at 2.54 25.4) (size 1.7 1.7) (drill 1) (layers *.Cu *.Mask) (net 33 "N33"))
  (pad "23" thru_hole oval (at 0 27.94) (size 1.7 1.7) (drill 1) (layers *.Cu *.Mask) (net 9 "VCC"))
  (pad "24" thru_hole oval (at 2.54 27.94) (size 1.7 1.7) (drill 1) (layers *.Cu *.Mask) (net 9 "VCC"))
  (pad "25" thru_hole oval (at 0 30.48) (size 1.7 1.7) (drill 1) (layers *.Cu *.Mask) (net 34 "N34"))
  (pad "26" thru_hole oval (at 2.54 30.48) (size 1.7 1.7) (drill 1) (layers *.Cu *.Mask) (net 34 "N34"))
  (pad "27" thru_hole oval (at 0 33.02) (size 1.7 1.7) (drill 1) (layers *.Cu *.Mask) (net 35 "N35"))
  (pad "28" thru_hole oval (at 2.54 33.02) (size 1.7 1.7) (drill 1) (layers *.Cu *.Mask) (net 35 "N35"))
  (pad "29" thru_hole oval (at 0 35.56) (size 1.7 1.7) (drill 1) (layers *.Cu *.Mask) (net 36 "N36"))
  (pad "30" thru_hole oval (at 2.54 35.56) (size 1.7 1.7) (drill 1) (layers *.Cu *.Mask) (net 36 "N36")))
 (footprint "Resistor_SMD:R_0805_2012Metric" (layer "F.Cu") (at 69.53 55.88 180)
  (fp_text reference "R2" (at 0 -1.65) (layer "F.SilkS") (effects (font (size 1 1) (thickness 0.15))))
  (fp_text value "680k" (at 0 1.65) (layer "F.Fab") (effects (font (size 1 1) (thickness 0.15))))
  (fp_line (start -0.227064 0.735) (end 0.227064 0.735) (layer "F.SilkS") (width 0.12))
  (fp_line (start -0.227064 -0.735) (end 0.227064 -0.735) (layer "F.SilkS") (width 0.12))
  (pad "1" smd roundrect (at -0.9125 0 180) (size 1.025 1.4) (layers "F.Cu" "F.Paste" "F.Mask") (roundrect_rratio 0.243902) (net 7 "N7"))
  (pad "2" smd roundrect (at 0.9125 0 180) (size 1.025 1.4) (layers "F.Cu" "F.Paste" "F.Mask") (roundrect_rratio 0.243902) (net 2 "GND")))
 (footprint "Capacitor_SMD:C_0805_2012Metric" (layer "F.Cu") (at 54.93 72.39)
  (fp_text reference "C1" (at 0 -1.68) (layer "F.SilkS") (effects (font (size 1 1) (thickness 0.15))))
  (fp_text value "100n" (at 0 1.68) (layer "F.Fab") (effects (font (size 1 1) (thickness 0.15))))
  (fp_line (start -0.261252 -0.735) (end 0.261252 -0.735) (layer "F.SilkS") (width 0.12))
  (fp_line (start -0.261252 0.735) (end 0.261252 0.735) (layer "F.SilkS") (width 0.12))
  (pad "1" smd roundrect (at -0.95 0) (size 1 1.45) (layers "F.Cu" "F.Paste" "F.Mask") (roundrect_rratio 0.25) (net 1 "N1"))
  (pad "2" smd roundrect (at 0.95 0) (size 1 1.45) (layers "F.Cu" "F.Paste" "F.Mask") (roundrect_rratio 0.25) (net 4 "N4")))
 (gr_rect (start 83.82 83.82) (end 36.83 20.32) (layer "Edge.Cuts") (width 0.05) (fill none))
 (segment (start 77.47 24.13) (end 80.01 24.13) (width 0.25) (layer "F.Cu") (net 23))
 (segment (start 80.01 26.67) (end 77.47 26.67) (width 0.25) (layer "F.Cu") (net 24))
 (segment (start 77.47 29.21) (end 80.01 29.21) (width 0.25) (layer "F.Cu") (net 25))
 (segment (start 80.01 31.75) (end 77.47 31.75) (width 0.25) (layer "F.Cu") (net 26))
 (segment (start 77.47 34.29) (end 80.01 34.29) (width 0.25) (layer "F.Cu") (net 27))
 (segment (start 80.01 36.83) (end 77.47 36.83) (width 0.25) (layer "F.Cu") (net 28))
 (segment (start 77.47 39.37) (end 80.01 39.37) (width 0.25) (layer "F.Cu") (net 29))
 (segment (start 80.01 41.91) (end 77.47 41.91) (width 0.25) (layer "F.Cu") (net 30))
 (segment (start 77.47 44.45) (end 80.01 44.45) (width 0.25) (layer "F.Cu") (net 31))
 (segment (start 80.01 46.99) (end 77.47 46.99) (width 0.25) (layer "F.Cu") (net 32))
 (segment (start 77.47 49.53) (end 80.01 49.53) (width 0.25) (layer "F.Cu") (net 33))
 (segment (start 64.705 71.755) (end 64.77 71.69) (width 0.25) (layer "F.Cu") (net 9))
 (segment (start 80.01 52.07) (end 77.47 52.07) (width 0.25) (layer "F.Cu") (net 9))
 (segment (start 64.77 71.69) (end 64.77 69.85) (width 0.25) (layer "F.Cu") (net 9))
 (via (at 64.77 69.85) (size 1.2) (drill 0.8) (layers "F.Cu" "B.Cu") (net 9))
 (segment (start 64.77 69.85) (end 64.77 62.23) (width 0.25) (layer "B.Cu") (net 9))
 (segment (start 74.93 52.07) (end 77.47 52.07) (width 0.25) (layer "B.Cu") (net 9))
 (segment (start 64.77 62.23) (end 74.93 52.07) (width 0.25) (layer "B.Cu") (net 9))
 (segment (start 77.47 54.61) (end 80.01 54.61) (width 0.25) (layer "F.Cu") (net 34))
 (segment (start 80.01 57.15) (end 77.47 57.15) (width 0.25) (layer "F.Cu") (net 35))
 (segment (start 77.47 59.69) (end 80.01 59.69) (width 0.25) (layer "F.Cu") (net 36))
 (segment (start 62.23 24.13) (end 59.69 24.13) (width 0.25) (layer "F.Cu") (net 10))
 (segment (start 59.69 26.67) (end 62.23 26.67) (width 0.25) (layer "F.Cu") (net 11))
 (segment (start 59.69 29.21) (end 62.23 29.21) (width 0.25) (layer "F.Cu") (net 12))
 (segment (start 62.23 31.75) (end 59.69 31.75) (width 0.25) (layer "F.Cu") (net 13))
 (segment (start 59.69 34.29) (end 62.23 34.29) (width 0.25) (layer "F.Cu") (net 14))
 (segment (start 62.23 36.83) (end 59.69 36.83) (width 0.25) (layer "F.Cu") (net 15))
 (segment (start 59.69 39.37) (end 62.23 39.37) (width 0.25) (layer "F.Cu") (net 16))
 (segment (start 62.23 41.91) (end 59.69 41.91) (width 0.25) (layer "F.Cu") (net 17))
 (segment (start 59.69 44.45) (end 62.23 44.45) (width 0.25) (layer "F.Cu") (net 18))
 (segment (start 62.23 46.99) (end 59.69 46.99) (width 0.25) (layer "F.Cu") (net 19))
 (segment (start 54.61 46.99) (end 57.15 49.53) (width 0.25) (layer "F.Cu") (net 5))
 (segment (start 59.755 74.295) (end 43.815 74.295) (width 0.25) (layer "F.Cu") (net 5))
 (segment (start 59.69 49.53) (end 62.23 49.53) (width 0.25) (layer "F.Cu") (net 5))
 (segment (start 45.71 26.66) (end 54.61 35.56) (width 0.25) (layer "F.Cu") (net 5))
 (segment (start 39.525 29.02) (end 41.885 26.66) (width 0.25) (layer "F.Cu") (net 5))
 (segment (start 57.15 49.53) (end 59.69 49.53) (width 0.25) (layer "F.Cu") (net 5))
 (segment (start 43.815 74.295) (end 39.525 70.005) (width 0.25) (layer "F.Cu") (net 5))
 (segment (start 54.61 35.56) (end 54.61 46.99) (width 0.25) (layer "F.Cu") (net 5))
 (segment (start 41.885 26.66) (end 45.71 26.66) (width 0.25) (layer "F.Cu") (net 5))
 (segment (start 39.525 70.005) (end 39.525 29.02) (width 0.25) (layer "F.Cu") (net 5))
 (segment (start 62.23 52.07) (end 68.58 52.07) (width 0.25) (layer "F.Cu") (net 2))
 (segment (start 59.755 75.565) (end 59.755 76.2) (width 0.25) (layer "F.Cu") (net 2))
 (segment (start 71.12 74.930698) (end 71.12 63.5) (width 0.25) (layer "F.Cu") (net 2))
 (segment (start 46.19 43.96) (end 46.19 50.33) (width 0.25) (layer "F.Cu") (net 2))
 (segment (start 46.19 50.33) (end 46.19 56.09) (width 0.25) (layer "F.Cu") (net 2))
 (segment (start 59.755 76.2) (end 61.025 77.47) (width 0.25) (layer "F.Cu") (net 2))
 (segment (start 68.58 55.8425) (end 68.6175 55.88) (width 0.25) (layer "F.Cu") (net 2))
 (segment (start 62.23 52.07) (end 59.69 52.07) (width 0.25) (layer "F.Cu") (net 2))
 (segment (start 68.58 52.07) (end 68.58 55.8425) (width 0.25) (layer "F.Cu") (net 2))
 (segment (start 68.6175 60.9975) (end 68.6175 55.88) (width 0.25) (layer "F.Cu") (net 2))
 (segment (start 61.025 77.47) (end 68.580698 77.47) (width 0.25) (layer "F.Cu") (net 2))
 (segment (start 68.580698 77.47) (end 71.12 74.930698) (width 0.25) (layer "F.Cu") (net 2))
 (segment (start 71.12 63.5) (end 68.6175 60.9975) (width 0.25) (layer "F.Cu") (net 2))
 (segment (start 55.67 56.09) (end 46.19 56.09) (width 0.25) (layer "B.Cu") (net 2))
 (segment (start 59.69 52.07) (end 55.67 56.09) (width 0.25) (layer "B.Cu") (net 2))
 (segment (start 59.69 54.61) (end 62.23 54.61) (width 0.25) (layer "F.Cu") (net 20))
 (segment (start 62.23 57.15) (end 59.69 57.15) (width 0.25) (layer "F.Cu") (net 21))
 (segment (start 59.69 59.69) (end 62.23 59.69) (width 0.25) (layer "F.Cu") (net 22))
 (segment (start 41.69 56.09) (end 41.69 69.63) (width 0.25) (layer "F.Cu") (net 1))
 (segment (start 41.69 69.63) (end 44.45 72.39) (width 0.25) (layer "F.Cu") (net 1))
 (segment (start 41.69 43.96) (end 41.69 56.09) (width 0.25) (layer "F.Cu") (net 1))
 (segment (start 44.45 72.39) (end 53.98 72.39) (width 0.25) (layer "F.Cu") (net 1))
 (segment (start 55.88 72.39) (end 56.515 73.025) (width 0.25) (layer "F.Cu") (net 4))
 (segment (start 56.515 73.025) (end 59.755 73.025) (width 0.25) (layer "F.Cu") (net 4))
 (segment (start 70.48 52.07) (end 70.4425 52.1075) (width 0.25) (layer "F.Cu") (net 7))
 (segment (start 70.4425 59.0975) (end 69.85 59.69) (width 0.25) (layer "F.Cu") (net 7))
 (segment (start 70.4425 55.88) (end 70.4425 59.0975) (width 0.25) (layer "F.Cu") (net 7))
 (segment (start 70.4425 52.1075) (end 70.4425 55.88) (width 0.25) (layer "F.Cu") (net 7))
 (segment (start 66.675 74.295) (end 64.705 74.295) (width 0.25) (layer "F.Cu") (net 7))
 (segment (start 67.31 73.66) (end 66.675 74.295) (width 0.25) (layer "F.Cu") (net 7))
 (via (at 69.85 59.69) (size 1.2) (drill 0.8) (layers "F.Cu" "B.Cu") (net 7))
 (via (at 67.31 73.66) (size 1.2) (drill 0.8) (layers "F.Cu" "B.Cu") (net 7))
 (segment (start 68.58 60.96) (end 69.85 59.69) (width 0.25) (layer "B.Cu") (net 7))
 (segment (start 68.58 72.39) (end 68.58 60.96) (width 0.25) (layer "B.Cu") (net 7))
 (segment (start 67.31 73.66) (end 68.58 72.39) (width 0.25) (layer "B.Cu") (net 7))
 (segment (start 41.885 34.28) (end 45.71 34.28) (width 0.25) (layer "F.Cu") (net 3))
 (segment (start 59.755 71.185) (end 59.755 71.755) (width 0.25) (layer "F.Cu") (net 3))
 (segment (start 54.61 69.85) (end 58.42 69.85) (width 0.25) (layer "F.Cu") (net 3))
 (segment (start 45.71 34.28) (end 50.8 39.37) (width 0.25) (layer "F.Cu") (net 3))
 (segment (start 50.8 39.37) (end 50.8 66.04) (width 0.25) (layer "F.Cu") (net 3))
 (segment (start 58.42 69.85) (end 59.755 71.185) (width 0.25) (layer "F.Cu") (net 3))
 (segment (start 50.8 66.04) (end 54.61 69.85) (width 0.25) (layer "F.Cu") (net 3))
 (segment (start 52.07 64.77) (end 54.61 67.31) (width 0.25) (layer "F.Cu") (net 8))
 (segment (start 41.885 31.74) (end 45.71 31.74) (width 0.25) (layer "F.Cu") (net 8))
 (segment (start 45.71 31.74) (end 52.07 38.1) (width 0.25) (layer "F.Cu") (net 8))
 (segment (start 66.04 67.31) (end 67.31 68.58) (width 0.25) (layer "F.Cu") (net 8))
 (segment (start 52.07 38.1) (end 52.07 64.77) (width 0.25) (layer "F.Cu") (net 8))
 (segment (start 67.31 71.755) (end 66.04 73.025) (width 0.25) (layer "F.Cu") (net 8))
 (segment (start 67.31 68.58) (end 67.31 71.755) (width 0.25) (layer "F.Cu") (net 8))
 (segment (start 54.61 67.31) (end 66.04 67.31) (width 0.25) (layer "F.Cu") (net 8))
 (segment (start 66.04 73.025) (end 64.705 73.025) (width 0.25) (layer "F.Cu") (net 8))
 (segment (start 68.58 75.565) (end 69.85 74.295) (width 0.25) (layer "F.Cu") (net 6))
 (segment (start 53.34 36.83) (end 45.71 29.2) (width 0.25) (layer "F.Cu") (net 6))
 (segment (start 53.34 63.5) (end 53.34 36.83) (width 0.25) (layer "F.Cu") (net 6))
 (segment (start 64.705 75.565) (end 68.58 75.565) (width 0.25) (layer "F.Cu") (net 6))
 (segment (start 45.71 29.2) (end 41.885 29.2) (width 0.25) (layer "F.Cu") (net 6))
 (segment (start 69.85 67.31) (end 68.58 66.04) (width 0.25) (layer "F.Cu") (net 6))
 (segment (start 69.85 74.295) (end 69.85 67.31) (width 0.25) (layer "F.Cu") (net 6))
 (segment (start 68.58 66.04) (end 55.88 66.04) (width 0.25) (layer "F.Cu") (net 6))
 (segment (start 55.88 66.04) (end 53.34 63.5) (width 0.25) (layer "F.Cu") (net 6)))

